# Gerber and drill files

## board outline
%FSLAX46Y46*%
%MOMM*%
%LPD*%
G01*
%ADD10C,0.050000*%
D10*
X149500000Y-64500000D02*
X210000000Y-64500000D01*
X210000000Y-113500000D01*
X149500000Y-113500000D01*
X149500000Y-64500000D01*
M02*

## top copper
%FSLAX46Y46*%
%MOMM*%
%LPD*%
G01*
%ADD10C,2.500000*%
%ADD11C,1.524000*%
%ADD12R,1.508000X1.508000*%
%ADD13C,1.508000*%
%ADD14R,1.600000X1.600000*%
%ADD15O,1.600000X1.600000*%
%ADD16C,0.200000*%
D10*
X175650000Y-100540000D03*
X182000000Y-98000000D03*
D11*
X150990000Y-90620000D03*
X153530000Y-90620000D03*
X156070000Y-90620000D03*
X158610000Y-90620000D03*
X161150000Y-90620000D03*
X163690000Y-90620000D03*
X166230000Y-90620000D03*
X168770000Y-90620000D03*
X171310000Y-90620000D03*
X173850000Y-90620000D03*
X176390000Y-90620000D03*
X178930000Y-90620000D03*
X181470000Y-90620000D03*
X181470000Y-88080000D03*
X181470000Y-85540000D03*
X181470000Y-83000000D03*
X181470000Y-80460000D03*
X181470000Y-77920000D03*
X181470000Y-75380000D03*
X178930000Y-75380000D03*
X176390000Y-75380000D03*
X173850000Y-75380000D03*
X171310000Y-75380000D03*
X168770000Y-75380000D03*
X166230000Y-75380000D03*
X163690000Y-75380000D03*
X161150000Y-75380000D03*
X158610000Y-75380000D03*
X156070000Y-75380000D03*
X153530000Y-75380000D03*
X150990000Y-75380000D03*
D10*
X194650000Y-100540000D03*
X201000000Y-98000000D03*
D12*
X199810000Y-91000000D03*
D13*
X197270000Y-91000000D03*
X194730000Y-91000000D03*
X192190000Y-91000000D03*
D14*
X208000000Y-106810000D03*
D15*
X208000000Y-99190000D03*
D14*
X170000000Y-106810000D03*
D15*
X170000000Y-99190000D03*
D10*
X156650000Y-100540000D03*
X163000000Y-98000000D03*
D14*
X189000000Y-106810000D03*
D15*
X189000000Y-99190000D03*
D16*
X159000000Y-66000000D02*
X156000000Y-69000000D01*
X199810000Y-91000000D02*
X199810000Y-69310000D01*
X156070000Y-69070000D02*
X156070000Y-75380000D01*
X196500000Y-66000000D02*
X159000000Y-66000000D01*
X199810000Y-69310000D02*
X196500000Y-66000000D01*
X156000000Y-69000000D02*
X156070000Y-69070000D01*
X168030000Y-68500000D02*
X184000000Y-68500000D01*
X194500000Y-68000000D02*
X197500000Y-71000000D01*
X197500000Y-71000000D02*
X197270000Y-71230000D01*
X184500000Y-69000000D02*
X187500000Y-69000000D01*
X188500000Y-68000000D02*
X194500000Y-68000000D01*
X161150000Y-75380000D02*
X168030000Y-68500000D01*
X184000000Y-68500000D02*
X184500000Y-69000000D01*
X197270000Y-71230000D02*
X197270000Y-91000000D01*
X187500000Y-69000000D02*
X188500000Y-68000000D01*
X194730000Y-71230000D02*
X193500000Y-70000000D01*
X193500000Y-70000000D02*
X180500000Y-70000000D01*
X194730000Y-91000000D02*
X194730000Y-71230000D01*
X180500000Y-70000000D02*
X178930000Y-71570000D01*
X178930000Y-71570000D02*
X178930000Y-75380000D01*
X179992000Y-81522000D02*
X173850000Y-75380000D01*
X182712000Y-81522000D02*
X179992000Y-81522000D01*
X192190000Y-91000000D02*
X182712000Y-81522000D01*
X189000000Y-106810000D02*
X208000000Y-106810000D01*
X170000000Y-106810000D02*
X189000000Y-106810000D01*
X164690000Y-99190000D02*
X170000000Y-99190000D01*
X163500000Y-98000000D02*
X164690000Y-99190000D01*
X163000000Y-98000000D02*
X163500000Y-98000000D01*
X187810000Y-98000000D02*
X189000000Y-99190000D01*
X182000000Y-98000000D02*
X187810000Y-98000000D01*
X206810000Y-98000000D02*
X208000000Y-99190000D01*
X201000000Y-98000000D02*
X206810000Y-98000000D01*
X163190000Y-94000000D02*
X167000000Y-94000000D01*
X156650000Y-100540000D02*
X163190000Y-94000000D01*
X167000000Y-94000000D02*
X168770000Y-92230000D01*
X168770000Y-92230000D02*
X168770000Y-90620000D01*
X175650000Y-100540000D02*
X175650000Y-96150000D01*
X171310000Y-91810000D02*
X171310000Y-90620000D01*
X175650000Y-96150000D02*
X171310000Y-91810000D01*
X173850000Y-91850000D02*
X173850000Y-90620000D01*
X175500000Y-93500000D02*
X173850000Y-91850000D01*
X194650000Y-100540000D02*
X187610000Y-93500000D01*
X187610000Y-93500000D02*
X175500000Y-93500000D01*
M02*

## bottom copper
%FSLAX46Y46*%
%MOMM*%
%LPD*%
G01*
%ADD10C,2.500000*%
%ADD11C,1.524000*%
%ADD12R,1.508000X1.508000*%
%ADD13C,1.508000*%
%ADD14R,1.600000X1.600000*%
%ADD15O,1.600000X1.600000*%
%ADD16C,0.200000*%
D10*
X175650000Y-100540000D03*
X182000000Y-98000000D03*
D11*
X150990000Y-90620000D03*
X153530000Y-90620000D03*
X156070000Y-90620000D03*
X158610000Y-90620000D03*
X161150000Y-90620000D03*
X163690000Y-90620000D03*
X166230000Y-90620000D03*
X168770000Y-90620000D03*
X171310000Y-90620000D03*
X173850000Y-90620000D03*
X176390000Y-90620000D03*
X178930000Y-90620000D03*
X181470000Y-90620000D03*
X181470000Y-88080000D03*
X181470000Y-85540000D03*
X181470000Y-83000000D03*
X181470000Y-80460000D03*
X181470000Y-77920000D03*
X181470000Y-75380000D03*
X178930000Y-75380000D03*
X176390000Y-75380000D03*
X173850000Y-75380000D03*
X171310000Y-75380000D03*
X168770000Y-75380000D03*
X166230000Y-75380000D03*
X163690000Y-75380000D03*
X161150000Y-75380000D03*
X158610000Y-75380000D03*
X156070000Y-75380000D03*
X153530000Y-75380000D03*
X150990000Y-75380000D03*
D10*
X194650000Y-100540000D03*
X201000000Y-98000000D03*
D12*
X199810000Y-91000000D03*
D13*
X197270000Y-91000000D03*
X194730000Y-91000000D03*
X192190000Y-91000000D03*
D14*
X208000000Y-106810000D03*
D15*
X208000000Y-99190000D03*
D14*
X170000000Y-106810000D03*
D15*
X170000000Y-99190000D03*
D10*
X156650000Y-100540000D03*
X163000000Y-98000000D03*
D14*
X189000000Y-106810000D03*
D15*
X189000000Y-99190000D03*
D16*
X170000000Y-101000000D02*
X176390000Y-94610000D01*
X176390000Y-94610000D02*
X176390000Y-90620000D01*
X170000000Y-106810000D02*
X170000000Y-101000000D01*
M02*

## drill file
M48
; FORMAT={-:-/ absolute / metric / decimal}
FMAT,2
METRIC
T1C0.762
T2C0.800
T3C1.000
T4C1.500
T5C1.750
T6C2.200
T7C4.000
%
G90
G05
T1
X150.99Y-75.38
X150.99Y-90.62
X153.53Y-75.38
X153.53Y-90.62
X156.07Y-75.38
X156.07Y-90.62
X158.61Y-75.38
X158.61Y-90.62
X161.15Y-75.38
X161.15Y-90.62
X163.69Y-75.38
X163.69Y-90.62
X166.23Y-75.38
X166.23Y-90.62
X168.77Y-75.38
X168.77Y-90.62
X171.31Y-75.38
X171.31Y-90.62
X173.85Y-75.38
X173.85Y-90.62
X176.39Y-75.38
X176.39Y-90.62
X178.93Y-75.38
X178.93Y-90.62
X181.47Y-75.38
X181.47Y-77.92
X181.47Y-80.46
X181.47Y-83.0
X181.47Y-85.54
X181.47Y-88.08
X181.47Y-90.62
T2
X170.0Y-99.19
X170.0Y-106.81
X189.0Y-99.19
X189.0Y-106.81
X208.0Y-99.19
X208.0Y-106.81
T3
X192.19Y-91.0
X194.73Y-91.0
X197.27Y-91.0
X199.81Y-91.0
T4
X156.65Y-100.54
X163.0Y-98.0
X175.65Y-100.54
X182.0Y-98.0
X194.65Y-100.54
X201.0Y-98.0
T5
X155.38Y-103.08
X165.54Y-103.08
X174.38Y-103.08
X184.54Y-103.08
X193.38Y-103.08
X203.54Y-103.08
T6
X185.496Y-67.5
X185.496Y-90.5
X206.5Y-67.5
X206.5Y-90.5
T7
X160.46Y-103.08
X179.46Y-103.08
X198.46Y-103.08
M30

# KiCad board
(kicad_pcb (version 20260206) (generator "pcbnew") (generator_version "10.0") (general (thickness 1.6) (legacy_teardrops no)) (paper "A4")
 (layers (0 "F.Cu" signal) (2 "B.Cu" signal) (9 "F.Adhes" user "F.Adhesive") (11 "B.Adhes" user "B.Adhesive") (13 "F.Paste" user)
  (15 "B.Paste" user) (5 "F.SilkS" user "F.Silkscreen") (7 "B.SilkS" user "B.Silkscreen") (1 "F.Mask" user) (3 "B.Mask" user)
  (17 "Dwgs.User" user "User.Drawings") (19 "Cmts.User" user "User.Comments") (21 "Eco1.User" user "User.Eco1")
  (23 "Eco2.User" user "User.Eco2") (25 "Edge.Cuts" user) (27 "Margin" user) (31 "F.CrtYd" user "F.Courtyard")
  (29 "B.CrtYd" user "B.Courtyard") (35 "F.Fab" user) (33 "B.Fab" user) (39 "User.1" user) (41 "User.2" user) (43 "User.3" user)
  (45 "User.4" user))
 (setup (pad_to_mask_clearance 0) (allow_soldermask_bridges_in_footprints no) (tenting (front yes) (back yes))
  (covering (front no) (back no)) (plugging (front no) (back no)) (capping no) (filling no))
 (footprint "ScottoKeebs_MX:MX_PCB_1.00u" (layer "F.Cu") (at 179.46 103.08)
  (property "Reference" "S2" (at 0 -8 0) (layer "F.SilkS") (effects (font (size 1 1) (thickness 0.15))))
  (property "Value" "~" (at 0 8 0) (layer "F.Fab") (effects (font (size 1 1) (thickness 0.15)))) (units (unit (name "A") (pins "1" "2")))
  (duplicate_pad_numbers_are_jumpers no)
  (pad "" np_thru_hole circle (at -5.08 0) (size 1.75 1.75) (drill 1.75) (layers "*.Cu" "*.Mask"))
  (pad "" np_thru_hole circle (at 0 0) (size 4 4) (drill 4) (layers "*.Cu" "*.Mask"))
  (pad "" np_thru_hole circle (at 5.08 0) (size 1.75 1.75) (drill 1.75) (layers "*.Cu" "*.Mask"))
  (pad "1" thru_hole circle (at -3.81 -2.54) (size 2.5 2.5) (drill 1.5) (layers "*.Cu" "*.Mask") (remove_unused_layers no)
   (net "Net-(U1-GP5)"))
  (pad "2" thru_hole circle (at 2.54 -5.08) (size 2.5 2.5) (drill 1.5) (layers "*.Cu" "*.Mask") (remove_unused_layers no) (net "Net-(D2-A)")))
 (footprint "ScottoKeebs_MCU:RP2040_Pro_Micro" (layer "F.Cu") (at 167.5 83 90)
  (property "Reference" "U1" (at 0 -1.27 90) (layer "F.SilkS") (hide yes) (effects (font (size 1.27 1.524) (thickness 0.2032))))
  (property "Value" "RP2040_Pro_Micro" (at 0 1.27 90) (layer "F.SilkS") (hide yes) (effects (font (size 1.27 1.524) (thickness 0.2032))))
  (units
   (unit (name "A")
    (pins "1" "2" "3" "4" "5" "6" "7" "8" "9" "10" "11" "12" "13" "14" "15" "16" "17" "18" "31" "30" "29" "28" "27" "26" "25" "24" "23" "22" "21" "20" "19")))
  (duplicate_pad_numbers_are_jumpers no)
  (pad "1" thru_hole circle (at -7.62 -16.51 90) (size 1.524 1.524) (drill 0.762) (layers "*.Cu" "*.Mask") (remove_unused_layers no)
   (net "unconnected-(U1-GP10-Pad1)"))
  (pad "2" thru_hole circle (at -7.62 -13.97 90) (size 1.524 1.524) (drill 0.762) (layers "*.Cu" "*.Mask") (remove_unused_layers no)
   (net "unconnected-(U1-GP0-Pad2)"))
  (pad "3" thru_hole circle (at -7.62 -11.43 90) (size 1.524 1.524) (drill 0.762) (layers "*.Cu" "*.Mask") (remove_unused_layers no)
   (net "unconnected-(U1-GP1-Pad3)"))
  (pad "4" thru_hole circle (at -7.62 -8.89 90) (size 1.524 1.524) (drill 0.762) (layers "*.Cu" "*.Mask") (remove_unused_layers no)
   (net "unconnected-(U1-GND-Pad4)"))
  (pad "5" thru_hole circle (at -7.62 -6.35 90) (size 1.524 1.524) (drill 0.762) (layers "*.Cu" "*.Mask") (remove_unused_layers no)
   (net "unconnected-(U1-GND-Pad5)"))
  (pad "6" thru_hole circle (at -7.62 -3.81 90) (size 1.524 1.524) (drill 0.762) (layers "*.Cu" "*.Mask") (remove_unused_layers no)
   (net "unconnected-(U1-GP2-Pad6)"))
  (pad "7" thru_hole circle (at -7.62 -1.27 90) (size 1.524 1.524) (drill 0.762) (layers "*.Cu" "*.Mask") (remove_unused_layers no)
   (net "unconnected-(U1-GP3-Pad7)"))
  (pad "8" thru_hole circle (at -7.62 1.27 90) (size 1.524 1.524) (drill 0.762) (layers "*.Cu" "*.Mask") (remove_unused_layers no)
   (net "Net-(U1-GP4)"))
  (pad "9" thru_hole circle (at -7.62 3.81 90) (size 1.524 1.524) (drill 0.762) (layers "*.Cu" "*.Mask") (remove_unused_layers no)
   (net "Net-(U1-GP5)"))
  (pad "10" thru_hole circle (at -7.62 6.35 90) (size 1.524 1.524) (drill 0.762) (layers "*.Cu" "*.Mask") (remove_unused_layers no)
   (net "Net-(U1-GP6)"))
  (pad "11" thru_hole circle (at -7.62 8.89 90) (size 1.524 1.524) (drill 0.762) (layers "*.Cu" "*.Mask") (remove_unused_layers no)
   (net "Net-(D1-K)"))
  (pad "12" thru_hole circle (at -7.62 11.43 90) (size 1.524 1.524) (drill 0.762) (layers "*.Cu" "*.Mask") (remove_unused_layers no)
   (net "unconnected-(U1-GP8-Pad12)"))
  (pad "13" thru_hole circle (at -7.62 13.97 90) (size 1.524 1.524) (drill 0.762) (layers "*.Cu" "*.Mask") (remove_unused_layers no)
   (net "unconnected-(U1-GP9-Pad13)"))
  (pad "14" thru_hole circle (at -5.08 13.97 90) (size 1.524 1.524) (drill 0.762) (layers "*.Cu" "*.Mask") (remove_unused_layers no)
   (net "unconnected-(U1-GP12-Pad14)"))
  (pad "15" thru_hole circle (at -2.54 13.97 90) (size 1.524 1.524) (drill 0.762) (layers "*.Cu" "*.Mask") (remove_unused_layers no)
   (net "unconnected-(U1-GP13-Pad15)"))
  (pad "16" thru_hole circle (at 0 13.97 90) (size 1.524 1.524) (drill 0.762) (layers "*.Cu" "*.Mask") (remove_unused_layers no)
   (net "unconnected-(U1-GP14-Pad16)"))
  (pad "17" thru_hole circle (at 2.54 13.97 90) (size 1.524 1.524) (drill 0.762) (layers "*.Cu" "*.Mask") (remove_unused_layers no)
   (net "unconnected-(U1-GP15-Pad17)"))
  (pad "18" thru_hole circle (at 5.08 13.97 90) (size 1.524 1.524) (drill 0.762) (layers "*.Cu" "*.Mask") (remove_unused_layers no)
   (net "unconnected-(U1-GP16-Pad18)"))
  (pad "19" thru_hole circle (at 7.62 13.97 90) (size 1.524 1.524) (drill 0.762) (layers "*.Cu" "*.Mask") (remove_unused_layers no)
   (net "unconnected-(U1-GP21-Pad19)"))
  (pad "20" thru_hole circle (at 7.62 11.43 90) (size 1.524 1.524) (drill 0.762) (layers "*.Cu" "*.Mask") (remove_unused_layers no)
   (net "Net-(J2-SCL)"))
  (pad "21" thru_hole circle (at 7.62 8.89 90) (size 1.524 1.524) (drill 0.762) (layers "*.Cu" "*.Mask") (remove_unused_layers no)
   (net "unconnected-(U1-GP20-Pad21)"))
  (pad "22" thru_hole circle (at 7.62 6.35 90) (size 1.524 1.524) (drill 0.762) (layers "*.Cu" "*.Mask") (remove_unused_layers no)
   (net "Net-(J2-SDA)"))
  (pad "23" thru_hole circle (at 7.62 3.81 90) (size 1.524 1.524) (drill 0.762) (layers "*.Cu" "*.Mask") (remove_unused_layers no)
   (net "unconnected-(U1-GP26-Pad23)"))
  (pad "24" thru_hole circle (at 7.62 1.27 90) (size 1.524 1.524) (drill 0.762) (layers "*.Cu" "*.Mask") (remove_unused_layers no)
   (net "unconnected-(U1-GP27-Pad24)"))
  (pad "25" thru_hole circle (at 7.62 -1.27 90) (size 1.524 1.524) (drill 0.762) (layers "*.Cu" "*.Mask") (remove_unused_layers no)
   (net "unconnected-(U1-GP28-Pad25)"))
  (pad "26" thru_hole circle (at 7.62 -3.81 90) (size 1.524 1.524) (drill 0.762) (layers "*.Cu" "*.Mask") (remove_unused_layers no)
   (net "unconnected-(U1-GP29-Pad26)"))
  (pad "27" thru_hole circle (at 7.62 -6.35 90) (size 1.524 1.524) (drill 0.762) (layers "*.Cu" "*.Mask") (remove_unused_layers no)
   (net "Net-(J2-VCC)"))
  (pad "28" thru_hole circle (at 7.62 -8.89 90) (size 1.524 1.524) (drill 0.762) (layers "*.Cu" "*.Mask") (remove_unused_layers no)
   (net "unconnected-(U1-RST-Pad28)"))
  (pad "29" thru_hole circle (at 7.62 -11.43 90) (size 1.524 1.524) (drill 0.762) (layers "*.Cu" "*.Mask") (remove_unused_layers no)
   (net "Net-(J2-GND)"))
  (pad "30" thru_hole circle (at 7.62 -13.97 90) (size 1.524 1.524) (drill 0.762) (layers "*.Cu" "*.Mask") (remove_unused_layers no)
   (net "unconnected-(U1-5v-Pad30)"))
  (pad "31" thru_hole circle (at 7.62 -16.51 90) (size 1.524 1.524) (drill 0.762) (layers "*.Cu" "*.Mask") (remove_unused_layers no)
   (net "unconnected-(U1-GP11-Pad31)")))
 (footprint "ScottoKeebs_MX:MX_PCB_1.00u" (layer "F.Cu") (at 198.46 103.08)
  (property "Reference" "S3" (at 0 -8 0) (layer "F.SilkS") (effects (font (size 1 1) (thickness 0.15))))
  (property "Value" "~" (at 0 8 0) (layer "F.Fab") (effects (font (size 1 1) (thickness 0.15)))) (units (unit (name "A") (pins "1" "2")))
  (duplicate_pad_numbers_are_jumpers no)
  (pad "" np_thru_hole circle (at -5.08 0) (size 1.75 1.75) (drill 1.75) (layers "*.Cu" "*.Mask"))
  (pad "" np_thru_hole circle (at 0 0) (size 4 4) (drill 4) (layers "*.Cu" "*.Mask"))
  (pad "" np_thru_hole circle (at 5.08 0) (size 1.75 1.75) (drill 1.75) (layers "*.Cu" "*.Mask"))
  (pad "1" thru_hole circle (at -3.81 -2.54) (size 2.5 2.5) (drill 1.5) (layers "*.Cu" "*.Mask") (remove_unused_layers no)
   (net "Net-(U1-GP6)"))
  (pad "2" thru_hole circle (at 2.54 -5.08) (size 2.5 2.5) (drill 1.5) (layers "*.Cu" "*.Mask") (remove_unused_layers no) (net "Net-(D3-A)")))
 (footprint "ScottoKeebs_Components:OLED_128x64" (layer "F.Cu") (at 196 79)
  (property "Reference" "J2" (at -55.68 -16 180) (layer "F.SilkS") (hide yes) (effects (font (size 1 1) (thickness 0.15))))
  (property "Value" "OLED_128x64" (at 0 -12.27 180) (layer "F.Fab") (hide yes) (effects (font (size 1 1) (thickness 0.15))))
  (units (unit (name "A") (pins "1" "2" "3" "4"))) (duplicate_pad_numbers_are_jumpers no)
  (pad "" np_thru_hole circle (at -10.50445 -11.5 180) (size 2.2 2.2) (drill 2.2) (layers "*.Cu" "*.Mask") (solder_mask_margin 0.102))
  (pad "" np_thru_hole circle (at -10.50445 11.5 180) (size 2.2 2.2) (drill 2.2) (layers "*.Cu" "*.Mask") (solder_mask_margin 0.102))
  (pad "" np_thru_hole circle (at 10.5 -11.5 180) (size 2.2 2.2) (drill 2.2) (layers "*.Cu" "*.Mask") (solder_mask_margin 0.102))
  (pad "" np_thru_hole circle (at 10.5 11.5 180) (size 2.2 2.2) (drill 2.2) (layers "*.Cu" "*.Mask") (solder_mask_margin 0.102))
  (pad "1" thru_hole rect (at 3.81 12 180) (size 1.508 1.508) (drill 1) (layers "*.Cu" "*.Mask") (remove_unused_layers no)
   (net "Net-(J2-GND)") (solder_mask_margin 0.102))
  (pad "2" thru_hole circle (at 1.27 12 180) (size 1.508 1.508) (drill 1) (layers "*.Cu" "*.Mask") (remove_unused_layers no)
   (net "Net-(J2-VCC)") (solder_mask_margin 0.102))
  (pad "3" thru_hole circle (at -1.27 12 180) (size 1.508 1.508) (drill 1) (layers "*.Cu" "*.Mask") (remove_unused_layers no)
   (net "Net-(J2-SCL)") (solder_mask_margin 0.102))
  (pad "4" thru_hole circle (at -3.81 12 180) (size 1.508 1.508) (drill 1) (layers "*.Cu" "*.Mask") (remove_unused_layers no)
   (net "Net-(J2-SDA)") (solder_mask_margin 0.102)))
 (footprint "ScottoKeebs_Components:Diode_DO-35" (layer "F.Cu") (at 208 106.81 90)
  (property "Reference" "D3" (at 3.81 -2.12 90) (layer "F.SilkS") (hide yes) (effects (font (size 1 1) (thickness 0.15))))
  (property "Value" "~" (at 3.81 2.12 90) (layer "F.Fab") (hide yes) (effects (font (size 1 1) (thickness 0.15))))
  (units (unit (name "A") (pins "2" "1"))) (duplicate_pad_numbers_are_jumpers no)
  (pad "1" thru_hole rect (at 0 0 90) (size 1.6 1.6) (drill 0.8) (layers "*.Cu" "*.Mask") (remove_unused_layers no) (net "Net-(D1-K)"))
  (pad "2" thru_hole oval (at 7.62 0 90) (size 1.6 1.6) (drill 0.8) (layers "*.Cu" "*.Mask") (remove_unused_layers no) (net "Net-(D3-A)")))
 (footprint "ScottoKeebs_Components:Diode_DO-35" (layer "F.Cu") (at 170 106.81 90)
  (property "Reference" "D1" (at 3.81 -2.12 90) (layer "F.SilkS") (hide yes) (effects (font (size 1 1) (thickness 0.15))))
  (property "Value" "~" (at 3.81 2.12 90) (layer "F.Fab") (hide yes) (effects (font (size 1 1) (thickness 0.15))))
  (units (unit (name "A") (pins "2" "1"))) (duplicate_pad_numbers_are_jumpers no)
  (pad "1" thru_hole rect (at 0 0 90) (size 1.6 1.6) (drill 0.8) (layers "*.Cu" "*.Mask") (remove_unused_layers no) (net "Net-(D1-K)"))
  (pad "2" thru_hole oval (at 7.62 0 90) (size 1.6 1.6) (drill 0.8) (layers "*.Cu" "*.Mask") (remove_unused_layers no) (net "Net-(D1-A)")))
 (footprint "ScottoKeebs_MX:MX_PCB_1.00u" (layer "F.Cu") (at 160.46 103.08)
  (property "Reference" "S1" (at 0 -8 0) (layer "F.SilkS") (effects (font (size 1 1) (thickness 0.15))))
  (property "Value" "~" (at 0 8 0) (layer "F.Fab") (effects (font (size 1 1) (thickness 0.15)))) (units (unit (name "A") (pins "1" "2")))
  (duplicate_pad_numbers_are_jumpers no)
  (pad "" np_thru_hole circle (at -5.08 0) (size 1.75 1.75) (drill 1.75) (layers "*.Cu" "*.Mask"))
  (pad "" np_thru_hole circle (at 0 0) (size 4 4) (drill 4) (layers "*.Cu" "*.Mask"))
  (pad "" np_thru_hole circle (at 5.08 0) (size 1.75 1.75) (drill 1.75) (layers "*.Cu" "*.Mask"))
  (pad "1" thru_hole circle (at -3.81 -2.54) (size 2.5 2.5) (drill 1.5) (layers "*.Cu" "*.Mask") (remove_unused_layers no)
   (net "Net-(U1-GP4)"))
  (pad "2" thru_hole circle (at 2.54 -5.08) (size 2.5 2.5) (drill 1.5) (layers "*.Cu" "*.Mask") (remove_unused_layers no) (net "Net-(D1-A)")))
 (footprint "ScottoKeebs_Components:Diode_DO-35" (layer "F.Cu") (at 189 106.81 90)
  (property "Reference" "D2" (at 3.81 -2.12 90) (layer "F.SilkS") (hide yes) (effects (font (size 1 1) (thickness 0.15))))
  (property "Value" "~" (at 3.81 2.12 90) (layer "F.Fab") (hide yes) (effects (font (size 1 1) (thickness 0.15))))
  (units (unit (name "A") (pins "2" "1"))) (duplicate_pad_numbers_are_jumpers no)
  (pad "1" thru_hole rect (at 0 0 90) (size 1.6 1.6) (drill 0.8) (layers "*.Cu" "*.Mask") (remove_unused_layers no) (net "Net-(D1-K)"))
  (pad "2" thru_hole oval (at 7.62 0 90) (size 1.6 1.6) (drill 0.8) (layers "*.Cu" "*.Mask") (remove_unused_layers no) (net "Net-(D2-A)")))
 (gr_rect (start 149.5 64.5) (end 210 113.5) (stroke (width 0.05) (type default)) (fill no) (layer "Edge.Cuts"))
 (segment (start 159 66) (end 156 69) (width 0.2) (layer "F.Cu") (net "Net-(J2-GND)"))
 (segment (start 199.81 91) (end 199.81 69.31) (width 0.2) (layer "F.Cu") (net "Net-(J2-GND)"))
 (segment (start 156.07 69.07) (end 156.07 75.38) (width 0.2) (layer "F.Cu") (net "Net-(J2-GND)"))
 (segment (start 196.5 66) (end 159 66) (width 0.2) (layer "F.Cu") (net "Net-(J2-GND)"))
 (segment (start 199.81 69.31) (end 196.5 66) (width 0.2) (layer "F.Cu") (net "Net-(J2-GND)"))
 (segment (start 156 69) (end 156.07 69.07) (width 0.2) (layer "F.Cu") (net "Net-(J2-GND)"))
 (segment (start 168.03 68.5) (end 184 68.5) (width 0.2) (layer "F.Cu") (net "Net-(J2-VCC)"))
 (segment (start 194.5 68) (end 197.5 71) (width 0.2) (layer "F.Cu") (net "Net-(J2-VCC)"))
 (segment (start 197.5 71) (end 197.27 71.23) (width 0.2) (layer "F.Cu") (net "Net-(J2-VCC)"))
 (segment (start 184.5 69) (end 187.5 69) (width 0.2) (layer "F.Cu") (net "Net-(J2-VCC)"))
 (segment (start 188.5 68) (end 194.5 68) (width 0.2) (layer "F.Cu") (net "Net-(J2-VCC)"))
 (segment (start 161.15 75.38) (end 168.03 68.5) (width 0.2) (layer "F.Cu") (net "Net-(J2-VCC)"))
 (segment (start 184 68.5) (end 184.5 69) (width 0.2) (layer "F.Cu") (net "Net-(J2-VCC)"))
 (segment (start 197.27 71.23) (end 197.27 91) (width 0.2) (layer "F.Cu") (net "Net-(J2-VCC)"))
 (segment (start 187.5 69) (end 188.5 68) (width 0.2) (layer "F.Cu") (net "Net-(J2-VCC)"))
 (segment (start 194.73 71.23) (end 193.5 70) (width 0.2) (layer "F.Cu") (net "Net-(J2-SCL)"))
 (segment (start 193.5 70) (end 180.5 70) (width 0.2) (layer "F.Cu") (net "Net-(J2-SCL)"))
 (segment (start 194.73 91) (end 194.73 71.23) (width 0.2) (layer "F.Cu") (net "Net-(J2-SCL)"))
 (segment (start 180.5 70) (end 178.93 71.57) (width 0.2) (layer "F.Cu") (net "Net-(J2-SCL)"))
 (segment (start 178.93 71.57) (end 178.93 75.38) (width 0.2) (layer "F.Cu") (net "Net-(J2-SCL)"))
 (segment (start 179.992 81.522) (end 173.85 75.38) (width 0.2) (layer "F.Cu") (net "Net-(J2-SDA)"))
 (segment (start 182.712 81.522) (end 179.992 81.522) (width 0.2) (layer "F.Cu") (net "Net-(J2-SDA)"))
 (segment (start 192.19 91) (end 182.712 81.522) (width 0.2) (layer "F.Cu") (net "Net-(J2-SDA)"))
 (segment (start 189 106.81) (end 208 106.81) (width 0.2) (layer "F.Cu") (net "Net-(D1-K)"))
 (segment (start 170 106.81) (end 189 106.81) (width 0.2) (layer "F.Cu") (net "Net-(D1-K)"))
 (segment (start 170 101) (end 176.39 94.61) (width 0.2) (layer "B.Cu") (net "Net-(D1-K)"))
 (segment (start 176.39 94.61) (end 176.39 90.62) (width 0.2) (layer "B.Cu") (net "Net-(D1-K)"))
 (segment (start 170 106.81) (end 170 101) (width 0.2) (layer "B.Cu") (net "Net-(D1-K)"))
 (segment (start 164.69 99.19) (end 170 99.19) (width 0.2) (layer "F.Cu") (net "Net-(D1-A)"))
 (segment (start 163.5 98) (end 164.69 99.19) (width 0.2) (layer "F.Cu") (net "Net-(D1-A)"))
 (segment (start 163 98) (end 163.5 98) (width 0.2) (layer "F.Cu") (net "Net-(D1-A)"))
 (segment (start 187.81 98) (end 189 99.19) (width 0.2) (layer "F.Cu") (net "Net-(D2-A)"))
 (segment (start 182 98) (end 187.81 98) (width 0.2) (layer "F.Cu") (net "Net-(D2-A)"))
 (segment (start 206.81 98) (end 208 99.19) (width 0.2) (layer "F.Cu") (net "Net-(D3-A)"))
 (segment (start 201 98) (end 206.81 98) (width 0.2) (layer "F.Cu") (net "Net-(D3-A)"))
 (segment (start 163.19 94) (end 167 94) (width 0.2) (layer "F.Cu") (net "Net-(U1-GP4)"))
 (segment (start 156.65 100.54) (end 163.19 94) (width 0.2) (layer "F.Cu") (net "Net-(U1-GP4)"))
 (segment (start 167 94) (end 168.77 92.23) (width 0.2) (layer "F.Cu") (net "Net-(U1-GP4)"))
 (segment (start 168.77 92.23) (end 168.77 90.62) (width 0.2) (layer "F.Cu") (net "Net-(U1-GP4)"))
 (segment (start 175.65 100.54) (end 175.65 96.15) (width 0.2) (layer "F.Cu") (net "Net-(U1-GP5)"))
 (segment (start 171.31 91.81) (end 171.31 90.62) (width 0.2) (layer "F.Cu") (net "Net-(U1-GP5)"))
 (segment (start 175.65 96.15) (end 171.31 91.81) (width 0.2) (layer "F.Cu") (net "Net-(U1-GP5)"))
 (segment (start 173.85 91.85) (end 173.85 90.62) (width 0.2) (layer "F.Cu") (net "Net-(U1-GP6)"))
 (segment (start 175.5 93.5) (end 173.85 91.85) (width 0.2) (layer "F.Cu") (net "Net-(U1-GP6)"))
 (segment (start 194.65 100.54) (end 187.61 93.5) (width 0.2) (layer "F.Cu") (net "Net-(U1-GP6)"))
 (segment (start 187.61 93.5) (end 175.5 93.5) (width 0.2) (layer "F.Cu") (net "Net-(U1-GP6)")))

